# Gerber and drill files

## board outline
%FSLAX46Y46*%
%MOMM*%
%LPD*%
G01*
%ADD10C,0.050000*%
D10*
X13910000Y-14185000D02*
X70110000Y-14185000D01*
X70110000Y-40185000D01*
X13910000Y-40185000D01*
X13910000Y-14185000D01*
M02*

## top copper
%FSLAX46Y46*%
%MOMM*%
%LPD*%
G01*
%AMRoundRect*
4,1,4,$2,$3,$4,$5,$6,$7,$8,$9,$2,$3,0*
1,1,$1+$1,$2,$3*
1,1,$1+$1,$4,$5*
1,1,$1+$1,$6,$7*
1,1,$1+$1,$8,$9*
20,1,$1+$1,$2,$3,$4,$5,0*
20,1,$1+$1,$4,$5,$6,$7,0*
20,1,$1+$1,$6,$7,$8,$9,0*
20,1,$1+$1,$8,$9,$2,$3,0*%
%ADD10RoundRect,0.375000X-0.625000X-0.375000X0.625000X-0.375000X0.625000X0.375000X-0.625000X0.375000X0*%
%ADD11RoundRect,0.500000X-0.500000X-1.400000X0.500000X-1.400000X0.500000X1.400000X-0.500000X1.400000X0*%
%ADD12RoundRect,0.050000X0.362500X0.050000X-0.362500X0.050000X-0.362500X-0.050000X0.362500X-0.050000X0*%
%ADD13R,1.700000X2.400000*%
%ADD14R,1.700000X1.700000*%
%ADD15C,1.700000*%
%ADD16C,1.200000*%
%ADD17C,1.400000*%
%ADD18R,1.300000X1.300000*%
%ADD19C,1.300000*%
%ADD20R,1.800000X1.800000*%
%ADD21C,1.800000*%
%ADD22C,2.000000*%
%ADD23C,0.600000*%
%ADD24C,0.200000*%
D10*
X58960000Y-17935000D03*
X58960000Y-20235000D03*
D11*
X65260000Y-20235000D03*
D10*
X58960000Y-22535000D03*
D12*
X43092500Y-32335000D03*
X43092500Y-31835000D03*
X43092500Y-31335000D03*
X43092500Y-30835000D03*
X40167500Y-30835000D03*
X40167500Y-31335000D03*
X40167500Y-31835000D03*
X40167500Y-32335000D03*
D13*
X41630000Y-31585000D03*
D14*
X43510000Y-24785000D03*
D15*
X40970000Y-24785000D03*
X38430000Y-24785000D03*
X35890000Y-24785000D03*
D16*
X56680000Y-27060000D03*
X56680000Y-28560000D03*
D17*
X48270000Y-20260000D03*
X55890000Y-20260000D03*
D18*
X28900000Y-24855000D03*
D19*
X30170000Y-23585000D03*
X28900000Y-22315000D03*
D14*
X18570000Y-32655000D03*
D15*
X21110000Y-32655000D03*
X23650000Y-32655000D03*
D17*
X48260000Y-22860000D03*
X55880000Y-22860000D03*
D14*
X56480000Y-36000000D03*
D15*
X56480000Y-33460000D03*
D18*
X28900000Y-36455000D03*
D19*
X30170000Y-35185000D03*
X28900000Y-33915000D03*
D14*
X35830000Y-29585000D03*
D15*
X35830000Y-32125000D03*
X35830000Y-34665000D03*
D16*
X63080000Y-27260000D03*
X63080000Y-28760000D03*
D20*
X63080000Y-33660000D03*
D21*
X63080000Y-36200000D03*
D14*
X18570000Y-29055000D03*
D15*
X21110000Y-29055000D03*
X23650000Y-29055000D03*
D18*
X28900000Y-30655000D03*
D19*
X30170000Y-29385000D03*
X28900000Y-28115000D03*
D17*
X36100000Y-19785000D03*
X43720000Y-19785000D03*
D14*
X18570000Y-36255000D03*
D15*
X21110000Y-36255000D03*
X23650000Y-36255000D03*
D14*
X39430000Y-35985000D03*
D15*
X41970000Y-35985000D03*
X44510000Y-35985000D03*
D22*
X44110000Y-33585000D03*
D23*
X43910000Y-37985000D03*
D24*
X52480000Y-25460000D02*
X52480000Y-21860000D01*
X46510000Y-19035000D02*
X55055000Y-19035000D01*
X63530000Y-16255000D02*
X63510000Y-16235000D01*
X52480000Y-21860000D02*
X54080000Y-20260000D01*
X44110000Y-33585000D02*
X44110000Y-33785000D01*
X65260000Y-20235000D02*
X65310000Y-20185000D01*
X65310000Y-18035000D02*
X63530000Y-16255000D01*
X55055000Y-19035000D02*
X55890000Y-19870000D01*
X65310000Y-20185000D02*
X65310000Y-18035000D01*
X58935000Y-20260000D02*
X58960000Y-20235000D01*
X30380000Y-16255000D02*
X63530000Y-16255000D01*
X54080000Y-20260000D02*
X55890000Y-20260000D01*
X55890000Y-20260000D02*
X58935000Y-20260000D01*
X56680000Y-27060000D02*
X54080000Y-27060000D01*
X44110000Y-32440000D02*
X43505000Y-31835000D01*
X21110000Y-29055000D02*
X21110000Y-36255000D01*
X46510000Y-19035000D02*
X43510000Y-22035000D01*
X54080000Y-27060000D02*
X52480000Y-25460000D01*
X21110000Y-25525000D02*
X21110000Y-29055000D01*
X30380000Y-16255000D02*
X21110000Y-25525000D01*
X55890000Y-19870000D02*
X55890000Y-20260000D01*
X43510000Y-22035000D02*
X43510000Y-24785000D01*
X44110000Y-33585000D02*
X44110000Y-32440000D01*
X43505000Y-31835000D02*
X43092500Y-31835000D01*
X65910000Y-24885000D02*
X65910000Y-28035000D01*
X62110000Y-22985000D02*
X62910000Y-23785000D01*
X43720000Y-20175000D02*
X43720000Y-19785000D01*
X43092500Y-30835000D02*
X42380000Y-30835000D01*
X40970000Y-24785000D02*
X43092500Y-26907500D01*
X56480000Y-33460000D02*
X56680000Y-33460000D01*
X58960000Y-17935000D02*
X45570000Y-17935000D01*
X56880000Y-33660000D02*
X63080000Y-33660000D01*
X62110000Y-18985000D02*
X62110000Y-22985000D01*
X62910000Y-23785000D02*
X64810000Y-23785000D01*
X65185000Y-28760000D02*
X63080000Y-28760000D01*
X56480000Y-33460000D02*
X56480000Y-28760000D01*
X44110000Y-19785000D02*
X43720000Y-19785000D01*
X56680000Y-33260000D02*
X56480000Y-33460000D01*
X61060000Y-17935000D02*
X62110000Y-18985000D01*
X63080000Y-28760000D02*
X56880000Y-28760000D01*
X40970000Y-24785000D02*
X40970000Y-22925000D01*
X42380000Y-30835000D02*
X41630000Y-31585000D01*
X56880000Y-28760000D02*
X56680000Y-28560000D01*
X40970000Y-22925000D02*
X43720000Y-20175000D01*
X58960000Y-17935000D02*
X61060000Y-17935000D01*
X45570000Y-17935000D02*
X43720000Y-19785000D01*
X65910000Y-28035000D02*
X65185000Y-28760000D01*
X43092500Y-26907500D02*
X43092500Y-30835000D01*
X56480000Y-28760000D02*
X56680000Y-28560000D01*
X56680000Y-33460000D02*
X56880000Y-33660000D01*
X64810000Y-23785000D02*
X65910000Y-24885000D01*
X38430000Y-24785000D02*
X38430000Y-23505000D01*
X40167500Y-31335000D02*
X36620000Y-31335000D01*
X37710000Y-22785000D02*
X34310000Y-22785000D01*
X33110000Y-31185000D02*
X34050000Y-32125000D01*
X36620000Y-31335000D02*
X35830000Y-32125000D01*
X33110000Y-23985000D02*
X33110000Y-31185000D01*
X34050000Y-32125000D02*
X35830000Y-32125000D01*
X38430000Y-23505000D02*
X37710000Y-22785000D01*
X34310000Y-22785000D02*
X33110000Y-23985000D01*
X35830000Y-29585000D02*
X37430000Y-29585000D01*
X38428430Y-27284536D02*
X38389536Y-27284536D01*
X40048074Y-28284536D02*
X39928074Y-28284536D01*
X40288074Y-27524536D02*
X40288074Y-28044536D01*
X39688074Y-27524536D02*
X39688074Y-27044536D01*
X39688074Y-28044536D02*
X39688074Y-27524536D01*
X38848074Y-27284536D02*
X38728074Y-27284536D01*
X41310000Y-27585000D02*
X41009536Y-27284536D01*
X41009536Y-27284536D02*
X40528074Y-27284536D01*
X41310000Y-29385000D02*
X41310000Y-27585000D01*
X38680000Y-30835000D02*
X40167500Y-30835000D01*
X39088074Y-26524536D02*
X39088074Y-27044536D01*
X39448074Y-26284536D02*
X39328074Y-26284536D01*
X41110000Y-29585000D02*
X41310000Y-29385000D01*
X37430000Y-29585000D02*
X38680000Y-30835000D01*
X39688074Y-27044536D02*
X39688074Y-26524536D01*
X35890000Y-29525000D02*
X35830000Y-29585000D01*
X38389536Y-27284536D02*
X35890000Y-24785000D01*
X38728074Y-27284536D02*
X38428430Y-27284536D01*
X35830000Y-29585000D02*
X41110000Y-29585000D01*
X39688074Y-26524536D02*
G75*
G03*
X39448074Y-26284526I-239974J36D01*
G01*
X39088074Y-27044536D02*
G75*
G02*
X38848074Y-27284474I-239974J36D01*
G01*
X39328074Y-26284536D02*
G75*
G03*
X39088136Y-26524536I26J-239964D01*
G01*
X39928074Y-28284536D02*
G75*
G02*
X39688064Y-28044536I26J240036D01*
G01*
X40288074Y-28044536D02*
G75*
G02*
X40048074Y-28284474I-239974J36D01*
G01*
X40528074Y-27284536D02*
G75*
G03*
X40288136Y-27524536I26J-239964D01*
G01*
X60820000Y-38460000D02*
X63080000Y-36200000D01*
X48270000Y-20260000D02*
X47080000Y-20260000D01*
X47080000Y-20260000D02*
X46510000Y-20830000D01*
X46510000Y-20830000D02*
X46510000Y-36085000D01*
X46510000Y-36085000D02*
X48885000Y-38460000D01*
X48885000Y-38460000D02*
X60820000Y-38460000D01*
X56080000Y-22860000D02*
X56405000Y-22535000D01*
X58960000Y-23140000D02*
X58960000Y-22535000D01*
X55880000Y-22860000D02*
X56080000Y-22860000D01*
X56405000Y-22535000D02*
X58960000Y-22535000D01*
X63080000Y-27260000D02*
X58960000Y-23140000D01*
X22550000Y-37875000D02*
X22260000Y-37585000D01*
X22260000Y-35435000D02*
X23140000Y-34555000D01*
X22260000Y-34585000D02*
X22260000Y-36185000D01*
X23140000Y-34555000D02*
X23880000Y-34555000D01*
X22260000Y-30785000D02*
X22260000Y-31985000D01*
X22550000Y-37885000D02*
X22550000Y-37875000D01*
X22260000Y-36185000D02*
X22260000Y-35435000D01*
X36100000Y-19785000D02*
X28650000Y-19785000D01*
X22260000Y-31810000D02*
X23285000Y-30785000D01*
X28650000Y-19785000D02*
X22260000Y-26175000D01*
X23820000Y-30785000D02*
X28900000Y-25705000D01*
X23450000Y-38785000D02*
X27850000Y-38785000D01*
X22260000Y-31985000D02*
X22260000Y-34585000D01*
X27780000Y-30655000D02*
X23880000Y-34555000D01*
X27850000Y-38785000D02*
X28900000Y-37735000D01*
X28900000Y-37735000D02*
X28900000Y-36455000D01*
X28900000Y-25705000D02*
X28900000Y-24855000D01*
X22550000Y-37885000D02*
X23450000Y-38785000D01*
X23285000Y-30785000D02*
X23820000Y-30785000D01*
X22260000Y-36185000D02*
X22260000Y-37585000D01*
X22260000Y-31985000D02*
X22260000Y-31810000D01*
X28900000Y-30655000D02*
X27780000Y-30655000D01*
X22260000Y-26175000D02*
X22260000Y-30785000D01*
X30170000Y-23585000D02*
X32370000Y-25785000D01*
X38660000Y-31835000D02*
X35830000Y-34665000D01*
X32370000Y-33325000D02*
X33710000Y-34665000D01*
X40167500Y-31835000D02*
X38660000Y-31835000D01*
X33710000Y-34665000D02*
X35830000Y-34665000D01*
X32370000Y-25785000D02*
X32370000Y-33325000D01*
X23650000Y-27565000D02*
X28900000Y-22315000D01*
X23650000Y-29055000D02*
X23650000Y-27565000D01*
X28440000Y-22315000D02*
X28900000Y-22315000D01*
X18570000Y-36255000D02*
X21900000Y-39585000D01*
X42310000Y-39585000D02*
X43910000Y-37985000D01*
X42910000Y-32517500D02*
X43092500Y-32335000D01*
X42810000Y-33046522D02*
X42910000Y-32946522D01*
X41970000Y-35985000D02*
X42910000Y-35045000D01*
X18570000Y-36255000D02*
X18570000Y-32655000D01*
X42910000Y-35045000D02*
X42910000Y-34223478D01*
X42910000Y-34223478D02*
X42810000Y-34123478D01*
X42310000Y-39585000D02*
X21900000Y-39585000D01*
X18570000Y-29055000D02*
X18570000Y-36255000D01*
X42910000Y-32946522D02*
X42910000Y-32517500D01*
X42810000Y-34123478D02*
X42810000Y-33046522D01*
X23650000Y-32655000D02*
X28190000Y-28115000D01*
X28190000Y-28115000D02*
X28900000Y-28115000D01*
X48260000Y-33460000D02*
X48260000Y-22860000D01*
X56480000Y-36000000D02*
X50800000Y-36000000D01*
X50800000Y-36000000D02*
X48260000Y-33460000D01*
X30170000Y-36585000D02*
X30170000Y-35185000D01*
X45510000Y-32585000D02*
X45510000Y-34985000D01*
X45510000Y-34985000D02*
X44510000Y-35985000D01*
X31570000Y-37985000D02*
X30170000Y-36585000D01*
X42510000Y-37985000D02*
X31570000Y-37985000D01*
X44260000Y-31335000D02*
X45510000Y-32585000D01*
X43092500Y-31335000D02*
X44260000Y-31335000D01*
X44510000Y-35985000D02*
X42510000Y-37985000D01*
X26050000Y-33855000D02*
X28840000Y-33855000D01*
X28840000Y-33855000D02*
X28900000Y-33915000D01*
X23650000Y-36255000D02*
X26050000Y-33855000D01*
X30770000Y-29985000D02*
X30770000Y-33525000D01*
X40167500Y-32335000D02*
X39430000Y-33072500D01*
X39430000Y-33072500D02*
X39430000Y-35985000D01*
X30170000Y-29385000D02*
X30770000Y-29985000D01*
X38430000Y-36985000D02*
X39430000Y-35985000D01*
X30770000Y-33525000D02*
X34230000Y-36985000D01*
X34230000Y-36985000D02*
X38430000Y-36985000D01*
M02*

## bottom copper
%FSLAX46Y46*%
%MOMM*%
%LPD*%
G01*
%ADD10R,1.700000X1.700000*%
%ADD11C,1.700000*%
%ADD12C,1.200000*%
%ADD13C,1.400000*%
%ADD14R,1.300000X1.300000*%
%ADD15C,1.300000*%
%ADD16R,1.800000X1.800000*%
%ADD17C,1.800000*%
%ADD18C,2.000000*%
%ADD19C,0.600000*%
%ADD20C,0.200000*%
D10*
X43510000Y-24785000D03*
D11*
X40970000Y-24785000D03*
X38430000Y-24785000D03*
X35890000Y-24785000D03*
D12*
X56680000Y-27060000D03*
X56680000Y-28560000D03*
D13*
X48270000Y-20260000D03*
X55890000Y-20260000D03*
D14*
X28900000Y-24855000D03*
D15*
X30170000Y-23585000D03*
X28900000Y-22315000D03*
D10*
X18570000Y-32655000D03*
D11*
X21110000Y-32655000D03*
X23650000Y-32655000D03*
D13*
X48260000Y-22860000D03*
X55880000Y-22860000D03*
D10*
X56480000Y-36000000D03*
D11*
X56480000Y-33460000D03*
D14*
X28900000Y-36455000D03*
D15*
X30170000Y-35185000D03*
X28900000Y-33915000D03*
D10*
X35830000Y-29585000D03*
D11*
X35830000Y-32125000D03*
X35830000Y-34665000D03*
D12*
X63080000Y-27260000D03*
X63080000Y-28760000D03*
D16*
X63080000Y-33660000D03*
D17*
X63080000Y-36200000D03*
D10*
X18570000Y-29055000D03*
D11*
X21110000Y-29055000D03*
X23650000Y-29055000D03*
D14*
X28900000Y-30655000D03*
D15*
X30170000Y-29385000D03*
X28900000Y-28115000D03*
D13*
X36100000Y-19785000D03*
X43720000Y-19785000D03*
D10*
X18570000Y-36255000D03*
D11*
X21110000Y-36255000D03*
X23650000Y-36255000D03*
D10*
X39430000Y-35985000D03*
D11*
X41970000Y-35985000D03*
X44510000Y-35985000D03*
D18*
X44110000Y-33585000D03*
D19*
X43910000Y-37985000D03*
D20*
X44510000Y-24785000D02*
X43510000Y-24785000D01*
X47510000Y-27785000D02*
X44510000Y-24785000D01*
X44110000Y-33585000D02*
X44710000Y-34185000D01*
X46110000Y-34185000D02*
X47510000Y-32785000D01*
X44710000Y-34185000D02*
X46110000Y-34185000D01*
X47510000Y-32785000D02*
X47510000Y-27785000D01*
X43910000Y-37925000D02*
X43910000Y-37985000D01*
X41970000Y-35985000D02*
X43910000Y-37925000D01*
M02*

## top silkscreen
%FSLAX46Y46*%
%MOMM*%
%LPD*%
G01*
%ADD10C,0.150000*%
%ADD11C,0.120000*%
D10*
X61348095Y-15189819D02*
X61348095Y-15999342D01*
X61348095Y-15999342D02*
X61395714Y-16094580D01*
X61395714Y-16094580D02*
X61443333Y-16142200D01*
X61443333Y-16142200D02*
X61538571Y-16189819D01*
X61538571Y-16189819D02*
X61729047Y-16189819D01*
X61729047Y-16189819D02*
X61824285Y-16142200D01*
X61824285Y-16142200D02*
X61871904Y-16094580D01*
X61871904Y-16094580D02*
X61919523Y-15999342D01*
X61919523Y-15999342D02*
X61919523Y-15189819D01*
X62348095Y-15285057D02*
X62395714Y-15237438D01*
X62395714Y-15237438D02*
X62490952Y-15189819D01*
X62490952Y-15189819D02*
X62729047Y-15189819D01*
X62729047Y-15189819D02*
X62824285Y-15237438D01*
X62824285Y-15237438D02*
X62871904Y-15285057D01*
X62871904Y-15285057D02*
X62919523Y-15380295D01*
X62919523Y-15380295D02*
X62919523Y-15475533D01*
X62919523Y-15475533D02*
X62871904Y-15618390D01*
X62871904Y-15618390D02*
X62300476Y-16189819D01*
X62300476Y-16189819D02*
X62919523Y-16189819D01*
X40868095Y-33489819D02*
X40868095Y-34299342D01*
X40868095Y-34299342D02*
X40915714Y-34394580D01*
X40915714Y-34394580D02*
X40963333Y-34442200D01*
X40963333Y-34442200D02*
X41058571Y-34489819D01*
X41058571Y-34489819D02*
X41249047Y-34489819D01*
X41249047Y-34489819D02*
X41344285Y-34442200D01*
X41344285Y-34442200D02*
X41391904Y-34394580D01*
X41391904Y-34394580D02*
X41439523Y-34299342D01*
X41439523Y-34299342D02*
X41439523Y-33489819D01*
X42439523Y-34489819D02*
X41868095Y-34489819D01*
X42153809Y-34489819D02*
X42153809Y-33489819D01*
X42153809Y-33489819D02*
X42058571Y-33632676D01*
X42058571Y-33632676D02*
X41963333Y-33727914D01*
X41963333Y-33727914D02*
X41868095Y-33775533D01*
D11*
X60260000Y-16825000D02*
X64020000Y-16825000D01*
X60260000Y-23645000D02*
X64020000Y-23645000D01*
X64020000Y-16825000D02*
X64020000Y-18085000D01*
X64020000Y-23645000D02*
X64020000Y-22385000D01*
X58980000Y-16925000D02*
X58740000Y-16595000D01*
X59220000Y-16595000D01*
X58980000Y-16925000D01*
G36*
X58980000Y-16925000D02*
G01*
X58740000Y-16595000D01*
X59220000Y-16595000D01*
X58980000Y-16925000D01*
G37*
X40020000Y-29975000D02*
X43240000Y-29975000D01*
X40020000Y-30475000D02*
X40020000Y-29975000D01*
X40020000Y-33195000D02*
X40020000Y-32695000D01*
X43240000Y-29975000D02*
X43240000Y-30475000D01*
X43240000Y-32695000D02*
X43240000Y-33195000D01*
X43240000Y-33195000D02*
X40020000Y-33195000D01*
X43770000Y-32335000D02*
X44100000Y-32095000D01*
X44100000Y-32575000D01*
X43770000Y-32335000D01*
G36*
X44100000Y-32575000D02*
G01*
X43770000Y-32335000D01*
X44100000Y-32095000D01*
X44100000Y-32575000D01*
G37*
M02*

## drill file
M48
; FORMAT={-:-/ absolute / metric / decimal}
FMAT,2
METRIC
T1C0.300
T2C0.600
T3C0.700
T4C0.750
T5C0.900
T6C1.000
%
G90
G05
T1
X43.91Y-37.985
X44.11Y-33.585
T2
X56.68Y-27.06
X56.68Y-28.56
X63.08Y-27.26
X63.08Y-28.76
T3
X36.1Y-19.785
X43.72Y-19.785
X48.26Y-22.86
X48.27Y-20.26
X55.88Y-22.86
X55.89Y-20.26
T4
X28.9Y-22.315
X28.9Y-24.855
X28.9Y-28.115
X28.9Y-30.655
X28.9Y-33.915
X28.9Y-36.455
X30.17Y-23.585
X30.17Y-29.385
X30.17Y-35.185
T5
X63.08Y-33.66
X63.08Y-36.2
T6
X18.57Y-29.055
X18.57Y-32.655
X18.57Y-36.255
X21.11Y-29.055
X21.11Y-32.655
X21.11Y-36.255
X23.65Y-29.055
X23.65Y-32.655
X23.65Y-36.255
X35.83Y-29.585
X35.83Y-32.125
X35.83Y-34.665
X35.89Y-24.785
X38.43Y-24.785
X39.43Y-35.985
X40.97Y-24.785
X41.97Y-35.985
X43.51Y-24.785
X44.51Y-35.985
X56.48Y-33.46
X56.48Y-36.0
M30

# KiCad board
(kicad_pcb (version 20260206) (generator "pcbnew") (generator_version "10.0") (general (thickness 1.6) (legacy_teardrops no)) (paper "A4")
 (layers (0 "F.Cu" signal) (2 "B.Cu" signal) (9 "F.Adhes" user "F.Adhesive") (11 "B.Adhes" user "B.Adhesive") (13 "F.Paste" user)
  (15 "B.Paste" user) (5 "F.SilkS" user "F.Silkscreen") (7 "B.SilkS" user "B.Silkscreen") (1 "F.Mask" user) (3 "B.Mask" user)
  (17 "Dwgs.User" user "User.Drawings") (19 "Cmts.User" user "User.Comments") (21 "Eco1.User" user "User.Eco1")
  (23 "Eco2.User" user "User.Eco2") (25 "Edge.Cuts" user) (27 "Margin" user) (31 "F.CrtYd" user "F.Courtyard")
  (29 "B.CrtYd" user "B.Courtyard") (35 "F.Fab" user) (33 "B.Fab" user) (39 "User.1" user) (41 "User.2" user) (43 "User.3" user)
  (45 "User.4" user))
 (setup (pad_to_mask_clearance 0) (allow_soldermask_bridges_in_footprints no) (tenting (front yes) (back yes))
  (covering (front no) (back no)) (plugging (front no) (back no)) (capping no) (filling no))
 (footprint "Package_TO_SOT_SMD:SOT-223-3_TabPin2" (layer "F.Cu") (at 62.11 20.235)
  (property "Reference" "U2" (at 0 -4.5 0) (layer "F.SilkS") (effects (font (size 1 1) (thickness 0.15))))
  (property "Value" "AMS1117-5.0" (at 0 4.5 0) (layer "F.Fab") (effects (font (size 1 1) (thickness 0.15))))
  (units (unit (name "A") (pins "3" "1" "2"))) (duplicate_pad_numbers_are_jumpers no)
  (fp_line (start -1.85 -3.41) (end 1.91 -3.41) (stroke (width 0.12) (type solid)) (layer "F.SilkS"))
  (fp_line (start -1.85 3.41) (end 1.91 3.41) (stroke (width 0.12) (type solid)) (layer "F.SilkS"))
  (fp_line (start 1.91 -3.41) (end 1.91 -2.15) (stroke (width 0.12) (type solid)) (layer "F.SilkS"))
  (fp_line (start 1.91 3.41) (end 1.91 2.15) (stroke (width 0.12) (type solid)) (layer "F.SilkS"))
  (fp_poly
   (pts (xy -3.13 -3.31) (xy -3.37 -3.64) (xy -2.89 -3.64) (xy -3.13 -3.31)) (stroke (width 0.12) (type solid)) (fill yes) (layer "F.SilkS"))
  (pad "1" smd roundrect (at -3.15 -2.3) (size 2 1.5) (layers "F.Cu" "F.Mask" "F.Paste") (roundrect_rratio 0.25) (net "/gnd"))
  (pad "2" smd roundrect (at -3.15 0) (size 2 1.5) (layers "F.Cu" "F.Mask" "F.Paste") (roundrect_rratio 0.25) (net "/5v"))
  (pad "2" smd roundrect (at 3.15 0) (size 2 3.8) (layers "F.Cu" "F.Mask" "F.Paste") (roundrect_rratio 0.25) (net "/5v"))
  (pad "3" smd roundrect (at -3.15 2.3) (size 2 1.5) (layers "F.Cu" "F.Mask" "F.Paste") (roundrect_rratio 0.25) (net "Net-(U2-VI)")))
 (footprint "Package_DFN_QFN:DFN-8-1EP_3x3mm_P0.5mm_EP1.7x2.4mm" (layer "F.Cu") (at 41.63 31.585 180)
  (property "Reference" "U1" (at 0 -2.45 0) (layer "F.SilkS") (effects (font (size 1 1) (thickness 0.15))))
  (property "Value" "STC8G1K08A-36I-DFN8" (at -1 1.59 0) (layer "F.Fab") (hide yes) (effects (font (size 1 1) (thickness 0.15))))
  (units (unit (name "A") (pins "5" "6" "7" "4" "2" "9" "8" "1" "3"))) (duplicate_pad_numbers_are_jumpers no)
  (fp_line (start 1.61 1.61) (end -1.61 1.61) (stroke (width 0.12) (type solid)) (layer "F.SilkS"))
  (fp_line (start 1.61 1.11) (end 1.61 1.61) (stroke (width 0.12) (type solid)) (layer "F.SilkS"))
  (fp_line (start 1.61 -1.61) (end 1.61 -1.11) (stroke (width 0.12) (type solid)) (layer "F.SilkS"))
  (fp_line (start -1.61 1.61) (end -1.61 1.11) (stroke (width 0.12) (type solid)) (layer "F.SilkS"))
  (fp_line (start -1.61 -1.11) (end -1.61 -1.61) (stroke (width 0.12) (type solid)) (layer "F.SilkS"))
  (fp_line (start -1.61 -1.61) (end 1.61 -1.61) (stroke (width 0.12) (type solid)) (layer "F.SilkS"))
  (fp_poly (pts (xy -2.14 -0.75) (xy -2.47 -0.51) (xy -2.47 -0.99)) (stroke (width 0.12) (type solid)) (fill yes) (layer "F.SilkS"))
  (pad "" smd roundrect (at 0 0 180) (size 1.37 1.93) (layers "F.Paste") (roundrect_rratio 0.182482))
  (pad "1" smd roundrect (at -1.4625 -0.75 180) (size 0.825 0.2) (layers "F.Cu" "F.Mask" "F.Paste") (roundrect_rratio 0.25) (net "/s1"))
  (pad "2" smd roundrect (at -1.4625 -0.25 180) (size 0.825 0.2) (layers "F.Cu" "F.Mask" "F.Paste") (roundrect_rratio 0.25) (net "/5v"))
  (pad "3" smd roundrect (at -1.4625 0.25 180) (size 0.825 0.2) (layers "F.Cu" "F.Mask" "F.Paste") (roundrect_rratio 0.25) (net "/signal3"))
  (pad "4" smd roundrect (at -1.4625 0.75 180) (size 0.825 0.2) (layers "F.Cu" "F.Mask" "F.Paste") (roundrect_rratio 0.25) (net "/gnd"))
  (pad "5" smd roundrect (at 1.4625 0.75 180) (size 0.825 0.2) (layers "F.Cu" "F.Mask" "F.Paste") (roundrect_rratio 0.25) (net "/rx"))
  (pad "6" smd roundrect (at 1.4625 0.25 180) (size 0.825 0.2) (layers "F.Cu" "F.Mask" "F.Paste") (roundrect_rratio 0.25) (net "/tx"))
  (pad "7" smd roundrect (at 1.4625 -0.25 180) (size 0.825 0.2) (layers "F.Cu" "F.Mask" "F.Paste") (roundrect_rratio 0.25) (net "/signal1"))
  (pad "8" smd roundrect (at 1.4625 -0.75 180) (size 0.825 0.2) (layers "F.Cu" "F.Mask" "F.Paste") (roundrect_rratio 0.25) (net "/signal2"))
  (pad "9" smd rect (at 0 0 180) (size 1.7 2.4) (layers "F.Cu" "F.Mask") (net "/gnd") (zone_connect 2)))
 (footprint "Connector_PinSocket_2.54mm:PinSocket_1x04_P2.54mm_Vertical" (layer "B.Cu") (at 43.51 24.785 90)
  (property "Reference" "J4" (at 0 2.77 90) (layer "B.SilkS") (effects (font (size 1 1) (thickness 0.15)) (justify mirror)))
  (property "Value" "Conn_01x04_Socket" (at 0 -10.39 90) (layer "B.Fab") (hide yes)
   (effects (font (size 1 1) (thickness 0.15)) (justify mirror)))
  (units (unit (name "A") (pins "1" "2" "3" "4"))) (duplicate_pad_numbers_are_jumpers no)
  (pad "1" thru_hole rect (at 0 0 90) (size 1.7 1.7) (drill 1) (layers "*.Cu" "*.Mask") (remove_unused_layers no) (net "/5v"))
  (pad "2" thru_hole circle (at 0 -2.54 90) (size 1.7 1.7) (drill 1) (layers "*.Cu" "*.Mask") (remove_unused_layers no) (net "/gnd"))
  (pad "3" thru_hole circle (at 0 -5.08 90) (size 1.7 1.7) (drill 1) (layers "*.Cu" "*.Mask") (remove_unused_layers no) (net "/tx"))
  (pad "4" thru_hole circle (at 0 -7.62 90) (size 1.7 1.7) (drill 1) (layers "*.Cu" "*.Mask") (remove_unused_layers no) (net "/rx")))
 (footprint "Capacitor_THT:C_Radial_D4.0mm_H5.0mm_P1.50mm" (layer "B.Cu") (at 56.68 27.06 -90)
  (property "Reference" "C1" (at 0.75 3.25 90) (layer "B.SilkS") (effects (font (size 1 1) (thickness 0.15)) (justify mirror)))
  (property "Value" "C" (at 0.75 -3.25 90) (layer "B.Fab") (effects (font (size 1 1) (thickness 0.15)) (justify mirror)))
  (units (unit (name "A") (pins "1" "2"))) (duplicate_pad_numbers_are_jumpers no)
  (pad "1" thru_hole circle (at 0 0 270) (size 1.2 1.2) (drill 0.6) (layers "*.Cu" "*.Mask") (remove_unused_layers no) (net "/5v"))
  (pad "2" thru_hole circle (at 1.5 0 270) (size 1.2 1.2) (drill 0.6) (layers "*.Cu" "*.Mask") (remove_unused_layers no) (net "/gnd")))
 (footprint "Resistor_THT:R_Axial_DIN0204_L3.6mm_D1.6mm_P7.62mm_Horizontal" (layer "B.Cu") (at 48.27 20.26)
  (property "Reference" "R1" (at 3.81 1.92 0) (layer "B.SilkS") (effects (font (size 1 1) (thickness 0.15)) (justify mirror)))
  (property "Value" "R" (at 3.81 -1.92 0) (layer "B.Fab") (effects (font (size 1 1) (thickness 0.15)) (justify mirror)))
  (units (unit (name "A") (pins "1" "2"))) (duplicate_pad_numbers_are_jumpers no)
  (pad "1" thru_hole circle (at 0 0) (size 1.4 1.4) (drill 0.7) (layers "*.Cu" "*.Mask") (remove_unused_layers no) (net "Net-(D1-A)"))
  (pad "2" thru_hole circle (at 7.62 0) (size 1.4 1.4) (drill 0.7) (layers "*.Cu" "*.Mask") (remove_unused_layers no) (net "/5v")))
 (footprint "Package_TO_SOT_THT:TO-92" (layer "B.Cu") (at 28.9 24.855 90)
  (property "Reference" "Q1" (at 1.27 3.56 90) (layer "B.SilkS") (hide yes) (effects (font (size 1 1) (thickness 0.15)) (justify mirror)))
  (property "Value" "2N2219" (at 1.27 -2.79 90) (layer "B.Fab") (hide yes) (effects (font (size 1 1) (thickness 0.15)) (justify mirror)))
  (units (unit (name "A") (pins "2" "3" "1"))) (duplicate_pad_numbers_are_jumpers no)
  (pad "1" thru_hole rect (at 0 0 90) (size 1.3 1.3) (drill 0.75) (layers "*.Cu" "*.Mask") (remove_unused_layers no) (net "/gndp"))
  (pad "2" thru_hole circle (at 1.27 1.27 90) (size 1.3 1.3) (drill 0.75) (layers "*.Cu" "*.Mask") (remove_unused_layers no)
   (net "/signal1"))
  (pad "3" thru_hole circle (at 2.54 0 90) (size 1.3 1.3) (drill 0.75) (layers "*.Cu" "*.Mask") (remove_unused_layers no) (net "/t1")))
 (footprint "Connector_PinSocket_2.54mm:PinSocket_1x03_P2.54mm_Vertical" (layer "B.Cu") (at 18.57 32.655 -90)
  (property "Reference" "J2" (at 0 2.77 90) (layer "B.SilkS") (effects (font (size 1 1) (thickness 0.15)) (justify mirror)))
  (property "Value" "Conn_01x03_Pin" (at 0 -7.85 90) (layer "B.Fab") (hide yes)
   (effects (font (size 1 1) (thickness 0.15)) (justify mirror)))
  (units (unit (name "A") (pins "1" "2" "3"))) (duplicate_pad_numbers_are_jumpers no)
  (pad "1" thru_hole rect (at 0 0 270) (size 1.7 1.7) (drill 1) (layers "*.Cu" "*.Mask") (remove_unused_layers no) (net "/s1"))
  (pad "2" thru_hole circle (at 0 -2.54 270) (size 1.7 1.7) (drill 1) (layers "*.Cu" "*.Mask") (remove_unused_layers no) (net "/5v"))
  (pad "3" thru_hole circle (at 0 -5.08 270) (size 1.7 1.7) (drill 1) (layers "*.Cu" "*.Mask") (remove_unused_layers no) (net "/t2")))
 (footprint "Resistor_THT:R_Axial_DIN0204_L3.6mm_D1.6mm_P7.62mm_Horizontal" (layer "B.Cu") (at 48.26 22.86)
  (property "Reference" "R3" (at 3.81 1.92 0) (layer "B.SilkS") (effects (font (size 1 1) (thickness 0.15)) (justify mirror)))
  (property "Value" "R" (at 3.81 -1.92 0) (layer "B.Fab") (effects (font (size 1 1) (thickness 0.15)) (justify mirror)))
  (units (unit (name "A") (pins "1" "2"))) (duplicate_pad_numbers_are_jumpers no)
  (pad "1" thru_hole circle (at 0 0) (size 1.4 1.4) (drill 0.7) (layers "*.Cu" "*.Mask") (remove_unused_layers no) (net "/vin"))
  (pad "2" thru_hole circle (at 7.62 0) (size 1.4 1.4) (drill 0.7) (layers "*.Cu" "*.Mask") (remove_unused_layers no) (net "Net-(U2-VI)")))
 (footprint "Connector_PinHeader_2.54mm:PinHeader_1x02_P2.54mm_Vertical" (layer "B.Cu") (at 56.48 36)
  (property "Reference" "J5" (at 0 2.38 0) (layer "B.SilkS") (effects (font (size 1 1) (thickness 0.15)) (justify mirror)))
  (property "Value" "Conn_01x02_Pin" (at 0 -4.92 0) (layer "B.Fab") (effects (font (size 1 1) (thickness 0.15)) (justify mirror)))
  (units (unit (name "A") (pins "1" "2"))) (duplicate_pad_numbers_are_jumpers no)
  (pad "1" thru_hole rect (at 0 0) (size 1.7 1.7) (drill 1) (layers "*.Cu" "*.Mask") (remove_unused_layers no) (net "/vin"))
  (pad "2" thru_hole circle (at 0 -2.54) (size 1.7 1.7) (drill 1) (layers "*.Cu" "*.Mask") (remove_unused_layers no) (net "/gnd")))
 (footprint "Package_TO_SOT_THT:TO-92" (layer "B.Cu") (at 28.9 36.455 90)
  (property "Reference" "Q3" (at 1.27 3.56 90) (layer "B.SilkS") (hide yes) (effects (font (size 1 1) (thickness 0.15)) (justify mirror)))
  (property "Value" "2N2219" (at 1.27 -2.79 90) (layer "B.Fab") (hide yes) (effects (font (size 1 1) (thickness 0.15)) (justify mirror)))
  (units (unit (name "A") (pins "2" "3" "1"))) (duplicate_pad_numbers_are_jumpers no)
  (pad "1" thru_hole rect (at 0 0 90) (size 1.3 1.3) (drill 0.75) (layers "*.Cu" "*.Mask") (remove_unused_layers no) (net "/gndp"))
  (pad "2" thru_hole circle (at 1.27 1.27 90) (size 1.3 1.3) (drill 0.75) (layers "*.Cu" "*.Mask") (remove_unused_layers no)
   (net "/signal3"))
  (pad "3" thru_hole circle (at 2.54 0 90) (size 1.3 1.3) (drill 0.75) (layers "*.Cu" "*.Mask") (remove_unused_layers no) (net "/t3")))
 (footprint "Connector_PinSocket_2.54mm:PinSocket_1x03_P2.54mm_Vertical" (layer "B.Cu") (at 35.83 29.585 180)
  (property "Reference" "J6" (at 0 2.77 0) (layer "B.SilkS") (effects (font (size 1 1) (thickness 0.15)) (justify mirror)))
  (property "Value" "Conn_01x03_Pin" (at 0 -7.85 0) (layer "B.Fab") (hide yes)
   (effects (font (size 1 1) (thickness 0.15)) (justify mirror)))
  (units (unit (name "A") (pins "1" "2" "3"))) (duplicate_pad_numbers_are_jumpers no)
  (pad "1" thru_hole rect (at 0 0 180) (size 1.7 1.7) (drill 1) (layers "*.Cu" "*.Mask") (remove_unused_layers no) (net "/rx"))
  (pad "2" thru_hole circle (at 0 -2.54 180) (size 1.7 1.7) (drill 1) (layers "*.Cu" "*.Mask") (remove_unused_layers no) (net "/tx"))
  (pad "3" thru_hole circle (at 0 -5.08 180) (size 1.7 1.7) (drill 1) (layers "*.Cu" "*.Mask") (remove_unused_layers no) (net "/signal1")))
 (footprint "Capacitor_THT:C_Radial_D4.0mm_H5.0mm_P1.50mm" (layer "B.Cu") (at 63.08 27.26 -90)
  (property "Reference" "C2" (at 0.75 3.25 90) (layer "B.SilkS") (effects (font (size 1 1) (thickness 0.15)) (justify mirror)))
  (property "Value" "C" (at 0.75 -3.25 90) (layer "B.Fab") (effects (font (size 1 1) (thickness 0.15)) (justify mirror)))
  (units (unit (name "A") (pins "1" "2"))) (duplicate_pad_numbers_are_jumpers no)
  (pad "1" thru_hole circle (at 0 0 270) (size 1.2 1.2) (drill 0.6) (layers "*.Cu" "*.Mask") (remove_unused_layers no) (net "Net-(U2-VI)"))
  (pad "2" thru_hole circle (at 1.5 0 270) (size 1.2 1.2) (drill 0.6) (layers "*.Cu" "*.Mask") (remove_unused_layers no) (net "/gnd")))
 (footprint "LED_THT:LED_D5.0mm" (layer "B.Cu") (at 63.08 33.66 -90)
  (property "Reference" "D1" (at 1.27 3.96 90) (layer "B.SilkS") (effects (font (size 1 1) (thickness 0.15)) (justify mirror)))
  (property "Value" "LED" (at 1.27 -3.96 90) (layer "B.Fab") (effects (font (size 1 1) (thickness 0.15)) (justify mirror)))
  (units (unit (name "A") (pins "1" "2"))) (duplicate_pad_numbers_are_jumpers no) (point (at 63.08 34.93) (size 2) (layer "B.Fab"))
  (pad "1" thru_hole rect (at 0 0 270) (size 1.8 1.8) (drill 0.9) (layers "*.Cu" "*.Mask") (remove_unused_layers no) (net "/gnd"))
  (pad "2" thru_hole circle (at 2.54 0 270) (size 1.8 1.8) (drill 0.9) (layers "*.Cu" "*.Mask") (remove_unused_layers no) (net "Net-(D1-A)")))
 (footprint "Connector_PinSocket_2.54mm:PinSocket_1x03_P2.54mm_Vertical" (layer "B.Cu") (at 18.57 29.055 -90)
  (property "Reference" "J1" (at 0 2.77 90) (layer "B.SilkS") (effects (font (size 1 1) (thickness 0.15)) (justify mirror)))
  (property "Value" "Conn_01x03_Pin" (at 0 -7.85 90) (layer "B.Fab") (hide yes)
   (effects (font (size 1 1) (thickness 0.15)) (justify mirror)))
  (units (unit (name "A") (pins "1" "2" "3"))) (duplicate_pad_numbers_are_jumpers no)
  (pad "1" thru_hole rect (at 0 0 270) (size 1.7 1.7) (drill 1) (layers "*.Cu" "*.Mask") (remove_unused_layers no) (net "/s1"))
  (pad "2" thru_hole circle (at 0 -2.54 270) (size 1.7 1.7) (drill 1) (layers "*.Cu" "*.Mask") (remove_unused_layers no) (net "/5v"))
  (pad "3" thru_hole circle (at 0 -5.08 270) (size 1.7 1.7) (drill 1) (layers "*.Cu" "*.Mask") (remove_unused_layers no) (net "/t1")))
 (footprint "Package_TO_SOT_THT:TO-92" (layer "B.Cu") (at 28.9 30.655 90)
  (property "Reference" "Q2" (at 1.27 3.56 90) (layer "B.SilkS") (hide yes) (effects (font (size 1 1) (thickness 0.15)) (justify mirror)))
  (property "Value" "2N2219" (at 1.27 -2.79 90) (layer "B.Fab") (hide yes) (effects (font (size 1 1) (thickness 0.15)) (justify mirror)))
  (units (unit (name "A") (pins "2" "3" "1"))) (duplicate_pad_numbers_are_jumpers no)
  (pad "1" thru_hole rect (at 0 0 90) (size 1.3 1.3) (drill 0.75) (layers "*.Cu" "*.Mask") (remove_unused_layers no) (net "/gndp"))
  (pad "2" thru_hole circle (at 1.27 1.27 90) (size 1.3 1.3) (drill 0.75) (layers "*.Cu" "*.Mask") (remove_unused_layers no)
   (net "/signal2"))
  (pad "3" thru_hole circle (at 2.54 0 90) (size 1.3 1.3) (drill 0.75) (layers "*.Cu" "*.Mask") (remove_unused_layers no) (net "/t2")))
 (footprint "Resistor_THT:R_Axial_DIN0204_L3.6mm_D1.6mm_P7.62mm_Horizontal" (layer "B.Cu") (at 36.1 19.785)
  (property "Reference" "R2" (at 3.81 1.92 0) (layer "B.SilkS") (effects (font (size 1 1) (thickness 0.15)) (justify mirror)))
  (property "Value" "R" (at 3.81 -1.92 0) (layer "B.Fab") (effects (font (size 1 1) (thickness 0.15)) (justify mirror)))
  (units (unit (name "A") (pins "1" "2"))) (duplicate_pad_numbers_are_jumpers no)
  (pad "1" thru_hole circle (at 0 0) (size 1.4 1.4) (drill 0.7) (layers "*.Cu" "*.Mask") (remove_unused_layers no) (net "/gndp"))
  (pad "2" thru_hole circle (at 7.62 0) (size 1.4 1.4) (drill 0.7) (layers "*.Cu" "*.Mask") (remove_unused_layers no) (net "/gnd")))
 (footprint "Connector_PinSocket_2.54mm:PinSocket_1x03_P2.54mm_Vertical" (layer "B.Cu") (at 18.57 36.255 -90)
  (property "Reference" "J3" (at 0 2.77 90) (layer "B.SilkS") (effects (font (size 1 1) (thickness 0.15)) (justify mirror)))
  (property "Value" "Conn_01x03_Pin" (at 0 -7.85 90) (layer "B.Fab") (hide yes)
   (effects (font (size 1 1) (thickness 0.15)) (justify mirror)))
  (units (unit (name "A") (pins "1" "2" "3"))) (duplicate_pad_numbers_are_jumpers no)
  (pad "1" thru_hole rect (at 0 0 270) (size 1.7 1.7) (drill 1) (layers "*.Cu" "*.Mask") (remove_unused_layers no) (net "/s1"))
  (pad "2" thru_hole circle (at 0 -2.54 270) (size 1.7 1.7) (drill 1) (layers "*.Cu" "*.Mask") (remove_unused_layers no) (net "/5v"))
  (pad "3" thru_hole circle (at 0 -5.08 270) (size 1.7 1.7) (drill 1) (layers "*.Cu" "*.Mask") (remove_unused_layers no) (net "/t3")))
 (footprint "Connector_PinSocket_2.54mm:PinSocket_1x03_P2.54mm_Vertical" (layer "B.Cu") (at 39.43 35.985 -90)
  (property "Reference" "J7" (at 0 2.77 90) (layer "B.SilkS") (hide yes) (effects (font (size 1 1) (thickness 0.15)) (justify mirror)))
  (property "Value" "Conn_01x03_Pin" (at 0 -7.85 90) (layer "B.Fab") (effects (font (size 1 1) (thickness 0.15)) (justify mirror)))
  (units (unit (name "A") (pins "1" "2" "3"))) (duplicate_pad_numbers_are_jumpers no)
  (pad "1" thru_hole rect (at 0 0 270) (size 1.7 1.7) (drill 1) (layers "*.Cu" "*.Mask") (remove_unused_layers no) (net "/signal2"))
  (pad "2" thru_hole circle (at 0 -2.54 270) (size 1.7 1.7) (drill 1) (layers "*.Cu" "*.Mask") (remove_unused_layers no) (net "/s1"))
  (pad "3" thru_hole circle (at 0 -5.08 270) (size 1.7 1.7) (drill 1) (layers "*.Cu" "*.Mask") (remove_unused_layers no) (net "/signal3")))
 (gr_rect (start 13.91 14.185) (end 70.11 40.185) (stroke (width 0.05) (type default)) (fill no) (layer "Edge.Cuts"))
 (segment (start 52.48 25.46) (end 52.48 21.86) (width 0.2) (layer "F.Cu") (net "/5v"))
 (segment (start 46.51 19.035) (end 55.055 19.035) (width 0.2) (layer "F.Cu") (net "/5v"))
 (segment (start 63.53 16.255) (end 63.51 16.235) (width 0.2) (layer "F.Cu") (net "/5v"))
 (segment (start 52.48 21.86) (end 54.08 20.26) (width 0.2) (layer "F.Cu") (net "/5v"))
 (segment (start 44.11 33.585) (end 44.11 33.785) (width 0.2) (layer "F.Cu") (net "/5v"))
 (segment (start 65.26 20.235) (end 65.31 20.185) (width 0.2) (layer "F.Cu") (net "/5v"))
 (segment (start 65.31 18.035) (end 63.53 16.255) (width 0.2) (layer "F.Cu") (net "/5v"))
 (segment (start 55.055 19.035) (end 55.89 19.87) (width 0.2) (layer "F.Cu") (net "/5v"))
 (segment (start 65.31 20.185) (end 65.31 18.035) (width 0.2) (layer "F.Cu") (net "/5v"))
 (segment (start 58.935 20.26) (end 58.96 20.235) (width 0.2) (layer "F.Cu") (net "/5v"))
 (segment (start 30.38 16.255) (end 63.53 16.255) (width 0.2) (layer "F.Cu") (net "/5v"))
 (segment (start 54.08 20.26) (end 55.89 20.26) (width 0.2) (layer "F.Cu") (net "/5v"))
 (segment (start 55.89 20.26) (end 58.935 20.26) (width 0.2) (layer "F.Cu") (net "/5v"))
 (segment (start 56.68 27.06) (end 54.08 27.06) (width 0.2) (layer "F.Cu") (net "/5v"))
 (segment (start 44.11 32.44) (end 43.505 31.835) (width 0.2) (layer "F.Cu") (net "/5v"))
 (segment (start 21.11 29.055) (end 21.11 36.255) (width 0.2) (layer "F.Cu") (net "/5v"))
 (segment (start 46.51 19.035) (end 43.51 22.035) (width 0.2) (layer "F.Cu") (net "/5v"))
 (segment (start 54.08 27.06) (end 52.48 25.46) (width 0.2) (layer "F.Cu") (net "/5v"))
 (segment (start 21.11 25.525) (end 21.11 29.055) (width 0.2) (layer "F.Cu") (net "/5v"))
 (segment (start 30.38 16.255) (end 21.11 25.525) (width 0.2) (layer "F.Cu") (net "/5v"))
 (segment (start 55.89 19.87) (end 55.89 20.26) (width 0.2) (layer "F.Cu") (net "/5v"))
 (segment (start 43.51 22.035) (end 43.51 24.785) (width 0.2) (layer "F.Cu") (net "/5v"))
 (segment (start 44.11 33.585) (end 44.11 32.44) (width 0.2) (layer "F.Cu") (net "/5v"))
 (segment (start 43.505 31.835) (end 43.0925 31.835) (width 0.2) (layer "F.Cu") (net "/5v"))
 (via (at 44.11 33.585) (size 2) (drill 0.3) (layers "F.Cu" "B.Cu") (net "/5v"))
 (segment (start 44.51 24.785) (end 43.51 24.785) (width 0.2) (layer "B.Cu") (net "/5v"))
 (segment (start 47.51 27.785) (end 44.51 24.785) (width 0.2) (layer "B.Cu") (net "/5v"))
 (segment (start 44.11 33.585) (end 44.71 34.185) (width 0.2) (layer "B.Cu") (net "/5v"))
 (segment (start 46.11 34.185) (end 47.51 32.785) (width 0.2) (layer "B.Cu") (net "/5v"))
 (segment (start 44.71 34.185) (end 46.11 34.185) (width 0.2) (layer "B.Cu") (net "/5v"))
 (segment (start 47.51 32.785) (end 47.51 27.785) (width 0.2) (layer "B.Cu") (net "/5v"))
 (segment (start 65.91 24.885) (end 65.91 28.035) (width 0.2) (layer "F.Cu") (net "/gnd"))
 (segment (start 62.11 22.985) (end 62.91 23.785) (width 0.2) (layer "F.Cu") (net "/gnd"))
 (segment (start 43.72 20.175) (end 43.72 19.785) (width 0.2) (layer "F.Cu") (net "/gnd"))
 (segment (start 43.0925 30.835) (end 42.38 30.835) (width 0.2) (layer "F.Cu") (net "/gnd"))
 (segment (start 40.97 24.785) (end 43.0925 26.9075) (width 0.2) (layer "F.Cu") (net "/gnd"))
 (segment (start 56.48 33.46) (end 56.68 33.46) (width 0.2) (layer "F.Cu") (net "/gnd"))
 (segment (start 58.96 17.935) (end 45.57 17.935) (width 0.2) (layer "F.Cu") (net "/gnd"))
 (segment (start 56.88 33.66) (end 63.08 33.66) (width 0.2) (layer "F.Cu") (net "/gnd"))
 (segment (start 62.11 18.985) (end 62.11 22.985) (width 0.2) (layer "F.Cu") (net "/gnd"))
 (segment (start 62.91 23.785) (end 64.81 23.785) (width 0.2) (layer "F.Cu") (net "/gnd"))
 (segment (start 65.185 28.76) (end 63.08 28.76) (width 0.2) (layer "F.Cu") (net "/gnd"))
 (segment (start 56.48 33.46) (end 56.48 28.76) (width 0.2) (layer "F.Cu") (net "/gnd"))
 (segment (start 44.11 19.785) (end 43.72 19.785) (width 0.2) (layer "F.Cu") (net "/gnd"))
 (segment (start 56.68 33.26) (end 56.48 33.46) (width 0.2) (layer "F.Cu") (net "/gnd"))
 (segment (start 61.06 17.935) (end 62.11 18.985) (width 0.2) (layer "F.Cu") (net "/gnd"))
 (segment (start 63.08 28.76) (end 56.88 28.76) (width 0.2) (layer "F.Cu") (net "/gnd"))
 (segment (start 40.97 24.785) (end 40.97 22.925) (width 0.2) (layer "F.Cu") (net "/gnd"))
 (segment (start 42.38 30.835) (end 41.63 31.585) (width 0.2) (layer "F.Cu") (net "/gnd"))
 (segment (start 56.88 28.76) (end 56.68 28.56) (width 0.2) (layer "F.Cu") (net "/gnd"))
 (segment (start 40.97 22.925) (end 43.72 20.175) (width 0.2) (layer "F.Cu") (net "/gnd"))
 (segment (start 58.96 17.935) (end 61.06 17.935) (width 0.2) (layer "F.Cu") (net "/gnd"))
 (segment (start 45.57 17.935) (end 43.72 19.785) (width 0.2) (layer "F.Cu") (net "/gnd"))
 (segment (start 65.91 28.035) (end 65.185 28.76) (width 0.2) (layer "F.Cu") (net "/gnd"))
 (segment (start 43.0925 26.9075) (end 43.0925 30.835) (width 0.2) (layer "F.Cu") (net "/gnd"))
 (segment (start 56.48 28.76) (end 56.68 28.56) (width 0.2) (layer "F.Cu") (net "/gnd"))
 (segment (start 56.68 33.46) (end 56.88 33.66) (width 0.2) (layer "F.Cu") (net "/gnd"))
 (segment (start 64.81 23.785) (end 65.91 24.885) (width 0.2) (layer "F.Cu") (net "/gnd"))
 (segment (start 38.43 24.785) (end 38.43 23.505) (width 0.2) (layer "F.Cu") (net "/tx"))
 (segment (start 40.1675 31.335) (end 36.62 31.335) (width 0.2) (layer "F.Cu") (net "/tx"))
 (segment (start 37.71 22.785) (end 34.31 22.785) (width 0.2) (layer "F.Cu") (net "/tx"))
 (segment (start 33.11 31.185) (end 34.05 32.125) (width 0.2) (layer "F.Cu") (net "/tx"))
 (segment (start 36.62 31.335) (end 35.83 32.125) (width 0.2) (layer "F.Cu") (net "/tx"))
 (segment (start 33.11 23.985) (end 33.11 31.185) (width 0.2) (layer "F.Cu") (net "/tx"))
 (segment (start 34.05 32.125) (end 35.83 32.125) (width 0.2) (layer "F.Cu") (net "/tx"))
 (segment (start 38.43 23.505) (end 37.71 22.785) (width 0.2) (layer "F.Cu") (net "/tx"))
 (segment (start 34.31 22.785) (end 33.11 23.985) (width 0.2) (layer "F.Cu") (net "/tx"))
 (segment (start 35.83 29.585) (end 37.43 29.585) (width 0.2) (layer "F.Cu") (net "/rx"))
 (segment (start 38.42843 27.284536) (end 38.389536 27.284536) (width 0.2) (layer "F.Cu") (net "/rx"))
 (segment (start 40.048074 28.284536) (end 39.928074 28.284536) (width 0.2) (layer "F.Cu") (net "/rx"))
 (segment (start 40.288074 27.524536) (end 40.288074 28.044536) (width 0.2) (layer "F.Cu") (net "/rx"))
 (segment (start 39.688074 27.524536) (end 39.688074 27.044536) (width 0.2) (layer "F.Cu") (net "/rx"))
 (segment (start 39.688074 28.044536) (end 39.688074 27.524536) (width 0.2) (layer "F.Cu") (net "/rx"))
 (segment (start 38.848074 27.284536) (end 38.728074 27.284536) (width 0.2) (layer "F.Cu") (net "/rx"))
 (segment (start 41.31 27.585) (end 41.009536 27.284536) (width 0.2) (layer "F.Cu") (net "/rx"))
 (segment (start 41.009536 27.284536) (end 40.528074 27.284536) (width 0.2) (layer "F.Cu") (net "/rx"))
 (segment (start 41.31 29.385) (end 41.31 27.585) (width 0.2) (layer "F.Cu") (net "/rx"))
 (segment (start 38.68 30.835) (end 40.1675 30.835) (width 0.2) (layer "F.Cu") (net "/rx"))
 (segment (start 39.088074 26.524536) (end 39.088074 27.044536) (width 0.2) (layer "F.Cu") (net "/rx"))
 (segment (start 39.448074 26.284536) (end 39.328074 26.284536) (width 0.2) (layer "F.Cu") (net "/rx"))
 (segment (start 41.11 29.585) (end 41.31 29.385) (width 0.2) (layer "F.Cu") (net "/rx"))
 (segment (start 37.43 29.585) (end 38.68 30.835) (width 0.2) (layer "F.Cu") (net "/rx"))
 (segment (start 39.688074 27.044536) (end 39.688074 26.524536) (width 0.2) (layer "F.Cu") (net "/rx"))
 (segment (start 35.89 29.525) (end 35.83 29.585) (width 0.2) (layer "F.Cu") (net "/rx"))
 (segment (start 38.389536 27.284536) (end 35.89 24.785) (width 0.2) (layer "F.Cu") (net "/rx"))
 (segment (start 38.728074 27.284536) (end 38.42843 27.284536) (width 0.2) (layer "F.Cu") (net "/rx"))
 (segment (start 35.83 29.585) (end 41.11 29.585) (width 0.2) (layer "F.Cu") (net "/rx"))
 (arc (start 39.688074 26.524536) (mid 39.61778 26.35483) (end 39.448074 26.284536) (width 0.2) (layer "F.Cu") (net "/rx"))
 (arc (start 39.088074 27.044536) (mid 39.01778 27.214242) (end 38.848074 27.284536) (width 0.2) (layer "F.Cu") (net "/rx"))
 (arc (start 39.328074 26.284536) (mid 39.158368 26.35483) (end 39.088074 26.524536) (width 0.2) (layer "F.Cu") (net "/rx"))
 (arc (start 39.928074 28.284536) (mid 39.758368 28.214242) (end 39.688074 28.044536) (width 0.2) (layer "F.Cu") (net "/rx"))
 (arc (start 40.288074 28.044536) (mid 40.21778 28.214242) (end 40.048074 28.284536) (width 0.2) (layer "F.Cu") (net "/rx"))
 (arc (start 40.528074 27.284536) (mid 40.358368 27.35483) (end 40.288074 27.524536) (width 0.2) (layer "F.Cu") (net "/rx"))
 (segment (start 60.82 38.46) (end 63.08 36.2) (width 0.2) (layer "F.Cu") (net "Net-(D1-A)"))
 (segment (start 48.27 20.26) (end 47.08 20.26) (width 0.2) (layer "F.Cu") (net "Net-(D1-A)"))
 (segment (start 47.08 20.26) (end 46.51 20.83) (width 0.2) (layer "F.Cu") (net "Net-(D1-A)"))
 (segment (start 46.51 20.83) (end 46.51 36.085) (width 0.2) (layer "F.Cu") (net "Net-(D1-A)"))
 (segment (start 46.51 36.085) (end 48.885 38.46) (width 0.2) (layer "F.Cu") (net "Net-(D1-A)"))
 (segment (start 48.885 38.46) (end 60.82 38.46) (width 0.2) (layer "F.Cu") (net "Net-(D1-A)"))
 (segment (start 56.08 22.86) (end 56.405 22.535) (width 0.2) (layer "F.Cu") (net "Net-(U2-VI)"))
 (segment (start 58.96 23.14) (end 58.96 22.535) (width 0.2) (layer "F.Cu") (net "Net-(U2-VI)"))
 (segment (start 55.88 22.86) (end 56.08 22.86) (width 0.2) (layer "F.Cu") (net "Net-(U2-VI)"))
 (segment (start 56.405 22.535) (end 58.96 22.535) (width 0.2) (layer "F.Cu") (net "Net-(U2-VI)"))
 (segment (start 63.08 27.26) (end 58.96 23.14) (width 0.2) (layer "F.Cu") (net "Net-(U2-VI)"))
 (segment (start 22.55 37.875) (end 22.26 37.585) (width 0.2) (layer "F.Cu") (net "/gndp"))
 (segment (start 22.26 35.435) (end 23.14 34.555) (width 0.2) (layer "F.Cu") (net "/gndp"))
 (segment (start 22.26 34.585) (end 22.26 36.185) (width 0.2) (layer "F.Cu") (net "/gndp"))
 (segment (start 23.14 34.555) (end 23.88 34.555) (width 0.2) (layer "F.Cu") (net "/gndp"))
 (segment (start 22.26 30.785) (end 22.26 31.985) (width 0.2) (layer "F.Cu") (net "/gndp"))
 (segment (start 22.55 37.885) (end 22.55 37.875) (width 0.2) (layer "F.Cu") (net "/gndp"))
 (segment (start 22.26 36.185) (end 22.26 35.435) (width 0.2) (layer "F.Cu") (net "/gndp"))
 (segment (start 36.1 19.785) (end 28.65 19.785) (width 0.2) (layer "F.Cu") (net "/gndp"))
 (segment (start 22.26 31.81) (end 23.285 30.785) (width 0.2) (layer "F.Cu") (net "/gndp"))
 (segment (start 28.65 19.785) (end 22.26 26.175) (width 0.2) (layer "F.Cu") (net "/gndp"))
 (segment (start 23.82 30.785) (end 28.9 25.705) (width 0.2) (layer "F.Cu") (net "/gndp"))
 (segment (start 23.45 38.785) (end 27.85 38.785) (width 0.2) (layer "F.Cu") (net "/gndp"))
 (segment (start 22.26 31.985) (end 22.26 34.585) (width 0.2) (layer "F.Cu") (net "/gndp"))
 (segment (start 27.78 30.655) (end 23.88 34.555) (width 0.2) (layer "F.Cu") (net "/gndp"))
 (segment (start 27.85 38.785) (end 28.9 37.735) (width 0.2) (layer "F.Cu") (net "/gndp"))
 (segment (start 28.9 37.735) (end 28.9 36.455) (width 0.2) (layer "F.Cu") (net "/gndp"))
 (segment (start 28.9 25.705) (end 28.9 24.855) (width 0.2) (layer "F.Cu") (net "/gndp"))
 (segment (start 22.55 37.885) (end 23.45 38.785) (width 0.2) (layer "F.Cu") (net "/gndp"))
 (segment (start 23.285 30.785) (end 23.82 30.785) (width 0.2) (layer "F.Cu") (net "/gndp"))
 (segment (start 22.26 36.185) (end 22.26 37.585) (width 0.2) (layer "F.Cu") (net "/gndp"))
 (segment (start 22.26 31.985) (end 22.26 31.81) (width 0.2) (layer "F.Cu") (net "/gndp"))
 (segment (start 28.9 30.655) (end 27.78 30.655) (width 0.2) (layer "F.Cu") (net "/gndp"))
 (segment (start 22.26 26.175) (end 22.26 30.785) (width 0.2) (layer "F.Cu") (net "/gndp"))
 (segment (start 30.17 23.585) (end 32.37 25.785) (width 0.2) (layer "F.Cu") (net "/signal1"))
 (segment (start 38.66 31.835) (end 35.83 34.665) (width 0.2) (layer "F.Cu") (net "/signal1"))
 (segment (start 32.37 33.325) (end 33.71 34.665) (width 0.2) (layer "F.Cu") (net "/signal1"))
 (segment (start 40.1675 31.835) (end 38.66 31.835) (width 0.2) (layer "F.Cu") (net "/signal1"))
 (segment (start 33.71 34.665) (end 35.83 34.665) (width 0.2) (layer "F.Cu") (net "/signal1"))
 (segment (start 32.37 25.785) (end 32.37 33.325) (width 0.2) (layer "F.Cu") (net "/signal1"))
 (segment (start 23.65 27.565) (end 28.9 22.315) (width 0.2) (layer "F.Cu") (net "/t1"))
 (segment (start 23.65 29.055) (end 23.65 27.565) (width 0.2) (layer "F.Cu") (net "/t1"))
 (segment (start 28.44 22.315) (end 28.9 22.315) (width 0.2) (layer "F.Cu") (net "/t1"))
 (segment (start 18.57 36.255) (end 21.9 39.585) (width 0.2) (layer "F.Cu") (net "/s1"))
 (segment (start 42.31 39.585) (end 43.91 37.985) (width 0.2) (layer "F.Cu") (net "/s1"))
 (segment (start 42.91 32.5175) (end 43.0925 32.335) (width 0.2) (layer "F.Cu") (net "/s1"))
 (segment (start 42.81 33.046522) (end 42.91 32.946522) (width 0.2) (layer "F.Cu") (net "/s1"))
 (segment (start 41.97 35.985) (end 42.91 35.045) (width 0.2) (layer "F.Cu") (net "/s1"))
 (segment (start 18.57 36.255) (end 18.57 32.655) (width 0.2) (layer "F.Cu") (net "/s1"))
 (segment (start 42.91 35.045) (end 42.91 34.223478) (width 0.2) (layer "F.Cu") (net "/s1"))
 (segment (start 42.91 34.223478) (end 42.81 34.123478) (width 0.2) (layer "F.Cu") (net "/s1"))
 (segment (start 42.31 39.585) (end 21.9 39.585) (width 0.2) (layer "F.Cu") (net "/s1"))
 (segment (start 18.57 29.055) (end 18.57 36.255) (width 0.2) (layer "F.Cu") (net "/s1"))
 (segment (start 42.91 32.946522) (end 42.91 32.5175) (width 0.2) (layer "F.Cu") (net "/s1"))
 (segment (start 42.81 34.123478) (end 42.81 33.046522) (width 0.2) (layer "F.Cu") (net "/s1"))
 (via (at 43.91 37.985) (size 0.6) (drill 0.3) (layers "F.Cu" "B.Cu") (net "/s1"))
 (segment (start 43.91 37.925) (end 43.91 37.985) (width 0.2) (layer "B.Cu") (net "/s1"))
 (segment (start 41.97 35.985) (end 43.91 37.925) (width 0.2) (layer "B.Cu") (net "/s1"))
 (segment (start 23.65 32.655) (end 28.19 28.115) (width 0.2) (layer "F.Cu") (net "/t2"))
 (segment (start 28.19 28.115) (end 28.9 28.115) (width 0.2) (layer "F.Cu") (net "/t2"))
 (segment (start 48.26 33.46) (end 48.26 22.86) (width 0.2) (layer "F.Cu") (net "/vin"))
 (segment (start 56.48 36) (end 50.8 36) (width 0.2) (layer "F.Cu") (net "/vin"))
 (segment (start 50.8 36) (end 48.26 33.46) (width 0.2) (layer "F.Cu") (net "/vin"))
 (segment (start 30.17 36.585) (end 30.17 35.185) (width 0.2) (layer "F.Cu") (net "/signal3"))
 (segment (start 45.51 32.585) (end 45.51 34.985) (width 0.2) (layer "F.Cu") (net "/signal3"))
 (segment (start 45.51 34.985) (end 44.51 35.985) (width 0.2) (layer "F.Cu") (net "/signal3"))
 (segment (start 31.57 37.985) (end 30.17 36.585) (width 0.2) (layer "F.Cu") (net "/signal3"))
 (segment (start 42.51 37.985) (end 31.57 37.985) (width 0.2) (layer "F.Cu") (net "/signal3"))
 (segment (start 44.26 31.335) (end 45.51 32.585) (width 0.2) (layer "F.Cu") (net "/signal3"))
 (segment (start 43.0925 31.335) (end 44.26 31.335) (width 0.2) (layer "F.Cu") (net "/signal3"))
 (segment (start 44.51 35.985) (end 42.51 37.985) (width 0.2) (layer "F.Cu") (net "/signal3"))
 (segment (start 26.05 33.855) (end 28.84 33.855) (width 0.2) (layer "F.Cu") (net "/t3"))
 (segment (start 28.84 33.855) (end 28.9 33.915) (width 0.2) (layer "F.Cu") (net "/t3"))
 (segment (start 23.65 36.255) (end 26.05 33.855) (width 0.2) (layer "F.Cu") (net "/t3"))
 (segment (start 30.77 29.985) (end 30.77 33.525) (width 0.2) (layer "F.Cu") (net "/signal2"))
 (segment (start 40.1675 32.335) (end 39.43 33.0725) (width 0.2) (layer "F.Cu") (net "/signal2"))
 (segment (start 39.43 33.0725) (end 39.43 35.985) (width 0.2) (layer "F.Cu") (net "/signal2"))
 (segment (start 30.17 29.385) (end 30.77 29.985) (width 0.2) (layer "F.Cu") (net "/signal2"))
 (segment (start 38.43 36.985) (end 39.43 35.985) (width 0.2) (layer "F.Cu") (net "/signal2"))
 (segment (start 30.77 33.525) (end 34.23 36.985) (width 0.2) (layer "F.Cu") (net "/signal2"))
 (segment (start 34.23 36.985) (end 38.43 36.985) (width 0.2) (layer "F.Cu") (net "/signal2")))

